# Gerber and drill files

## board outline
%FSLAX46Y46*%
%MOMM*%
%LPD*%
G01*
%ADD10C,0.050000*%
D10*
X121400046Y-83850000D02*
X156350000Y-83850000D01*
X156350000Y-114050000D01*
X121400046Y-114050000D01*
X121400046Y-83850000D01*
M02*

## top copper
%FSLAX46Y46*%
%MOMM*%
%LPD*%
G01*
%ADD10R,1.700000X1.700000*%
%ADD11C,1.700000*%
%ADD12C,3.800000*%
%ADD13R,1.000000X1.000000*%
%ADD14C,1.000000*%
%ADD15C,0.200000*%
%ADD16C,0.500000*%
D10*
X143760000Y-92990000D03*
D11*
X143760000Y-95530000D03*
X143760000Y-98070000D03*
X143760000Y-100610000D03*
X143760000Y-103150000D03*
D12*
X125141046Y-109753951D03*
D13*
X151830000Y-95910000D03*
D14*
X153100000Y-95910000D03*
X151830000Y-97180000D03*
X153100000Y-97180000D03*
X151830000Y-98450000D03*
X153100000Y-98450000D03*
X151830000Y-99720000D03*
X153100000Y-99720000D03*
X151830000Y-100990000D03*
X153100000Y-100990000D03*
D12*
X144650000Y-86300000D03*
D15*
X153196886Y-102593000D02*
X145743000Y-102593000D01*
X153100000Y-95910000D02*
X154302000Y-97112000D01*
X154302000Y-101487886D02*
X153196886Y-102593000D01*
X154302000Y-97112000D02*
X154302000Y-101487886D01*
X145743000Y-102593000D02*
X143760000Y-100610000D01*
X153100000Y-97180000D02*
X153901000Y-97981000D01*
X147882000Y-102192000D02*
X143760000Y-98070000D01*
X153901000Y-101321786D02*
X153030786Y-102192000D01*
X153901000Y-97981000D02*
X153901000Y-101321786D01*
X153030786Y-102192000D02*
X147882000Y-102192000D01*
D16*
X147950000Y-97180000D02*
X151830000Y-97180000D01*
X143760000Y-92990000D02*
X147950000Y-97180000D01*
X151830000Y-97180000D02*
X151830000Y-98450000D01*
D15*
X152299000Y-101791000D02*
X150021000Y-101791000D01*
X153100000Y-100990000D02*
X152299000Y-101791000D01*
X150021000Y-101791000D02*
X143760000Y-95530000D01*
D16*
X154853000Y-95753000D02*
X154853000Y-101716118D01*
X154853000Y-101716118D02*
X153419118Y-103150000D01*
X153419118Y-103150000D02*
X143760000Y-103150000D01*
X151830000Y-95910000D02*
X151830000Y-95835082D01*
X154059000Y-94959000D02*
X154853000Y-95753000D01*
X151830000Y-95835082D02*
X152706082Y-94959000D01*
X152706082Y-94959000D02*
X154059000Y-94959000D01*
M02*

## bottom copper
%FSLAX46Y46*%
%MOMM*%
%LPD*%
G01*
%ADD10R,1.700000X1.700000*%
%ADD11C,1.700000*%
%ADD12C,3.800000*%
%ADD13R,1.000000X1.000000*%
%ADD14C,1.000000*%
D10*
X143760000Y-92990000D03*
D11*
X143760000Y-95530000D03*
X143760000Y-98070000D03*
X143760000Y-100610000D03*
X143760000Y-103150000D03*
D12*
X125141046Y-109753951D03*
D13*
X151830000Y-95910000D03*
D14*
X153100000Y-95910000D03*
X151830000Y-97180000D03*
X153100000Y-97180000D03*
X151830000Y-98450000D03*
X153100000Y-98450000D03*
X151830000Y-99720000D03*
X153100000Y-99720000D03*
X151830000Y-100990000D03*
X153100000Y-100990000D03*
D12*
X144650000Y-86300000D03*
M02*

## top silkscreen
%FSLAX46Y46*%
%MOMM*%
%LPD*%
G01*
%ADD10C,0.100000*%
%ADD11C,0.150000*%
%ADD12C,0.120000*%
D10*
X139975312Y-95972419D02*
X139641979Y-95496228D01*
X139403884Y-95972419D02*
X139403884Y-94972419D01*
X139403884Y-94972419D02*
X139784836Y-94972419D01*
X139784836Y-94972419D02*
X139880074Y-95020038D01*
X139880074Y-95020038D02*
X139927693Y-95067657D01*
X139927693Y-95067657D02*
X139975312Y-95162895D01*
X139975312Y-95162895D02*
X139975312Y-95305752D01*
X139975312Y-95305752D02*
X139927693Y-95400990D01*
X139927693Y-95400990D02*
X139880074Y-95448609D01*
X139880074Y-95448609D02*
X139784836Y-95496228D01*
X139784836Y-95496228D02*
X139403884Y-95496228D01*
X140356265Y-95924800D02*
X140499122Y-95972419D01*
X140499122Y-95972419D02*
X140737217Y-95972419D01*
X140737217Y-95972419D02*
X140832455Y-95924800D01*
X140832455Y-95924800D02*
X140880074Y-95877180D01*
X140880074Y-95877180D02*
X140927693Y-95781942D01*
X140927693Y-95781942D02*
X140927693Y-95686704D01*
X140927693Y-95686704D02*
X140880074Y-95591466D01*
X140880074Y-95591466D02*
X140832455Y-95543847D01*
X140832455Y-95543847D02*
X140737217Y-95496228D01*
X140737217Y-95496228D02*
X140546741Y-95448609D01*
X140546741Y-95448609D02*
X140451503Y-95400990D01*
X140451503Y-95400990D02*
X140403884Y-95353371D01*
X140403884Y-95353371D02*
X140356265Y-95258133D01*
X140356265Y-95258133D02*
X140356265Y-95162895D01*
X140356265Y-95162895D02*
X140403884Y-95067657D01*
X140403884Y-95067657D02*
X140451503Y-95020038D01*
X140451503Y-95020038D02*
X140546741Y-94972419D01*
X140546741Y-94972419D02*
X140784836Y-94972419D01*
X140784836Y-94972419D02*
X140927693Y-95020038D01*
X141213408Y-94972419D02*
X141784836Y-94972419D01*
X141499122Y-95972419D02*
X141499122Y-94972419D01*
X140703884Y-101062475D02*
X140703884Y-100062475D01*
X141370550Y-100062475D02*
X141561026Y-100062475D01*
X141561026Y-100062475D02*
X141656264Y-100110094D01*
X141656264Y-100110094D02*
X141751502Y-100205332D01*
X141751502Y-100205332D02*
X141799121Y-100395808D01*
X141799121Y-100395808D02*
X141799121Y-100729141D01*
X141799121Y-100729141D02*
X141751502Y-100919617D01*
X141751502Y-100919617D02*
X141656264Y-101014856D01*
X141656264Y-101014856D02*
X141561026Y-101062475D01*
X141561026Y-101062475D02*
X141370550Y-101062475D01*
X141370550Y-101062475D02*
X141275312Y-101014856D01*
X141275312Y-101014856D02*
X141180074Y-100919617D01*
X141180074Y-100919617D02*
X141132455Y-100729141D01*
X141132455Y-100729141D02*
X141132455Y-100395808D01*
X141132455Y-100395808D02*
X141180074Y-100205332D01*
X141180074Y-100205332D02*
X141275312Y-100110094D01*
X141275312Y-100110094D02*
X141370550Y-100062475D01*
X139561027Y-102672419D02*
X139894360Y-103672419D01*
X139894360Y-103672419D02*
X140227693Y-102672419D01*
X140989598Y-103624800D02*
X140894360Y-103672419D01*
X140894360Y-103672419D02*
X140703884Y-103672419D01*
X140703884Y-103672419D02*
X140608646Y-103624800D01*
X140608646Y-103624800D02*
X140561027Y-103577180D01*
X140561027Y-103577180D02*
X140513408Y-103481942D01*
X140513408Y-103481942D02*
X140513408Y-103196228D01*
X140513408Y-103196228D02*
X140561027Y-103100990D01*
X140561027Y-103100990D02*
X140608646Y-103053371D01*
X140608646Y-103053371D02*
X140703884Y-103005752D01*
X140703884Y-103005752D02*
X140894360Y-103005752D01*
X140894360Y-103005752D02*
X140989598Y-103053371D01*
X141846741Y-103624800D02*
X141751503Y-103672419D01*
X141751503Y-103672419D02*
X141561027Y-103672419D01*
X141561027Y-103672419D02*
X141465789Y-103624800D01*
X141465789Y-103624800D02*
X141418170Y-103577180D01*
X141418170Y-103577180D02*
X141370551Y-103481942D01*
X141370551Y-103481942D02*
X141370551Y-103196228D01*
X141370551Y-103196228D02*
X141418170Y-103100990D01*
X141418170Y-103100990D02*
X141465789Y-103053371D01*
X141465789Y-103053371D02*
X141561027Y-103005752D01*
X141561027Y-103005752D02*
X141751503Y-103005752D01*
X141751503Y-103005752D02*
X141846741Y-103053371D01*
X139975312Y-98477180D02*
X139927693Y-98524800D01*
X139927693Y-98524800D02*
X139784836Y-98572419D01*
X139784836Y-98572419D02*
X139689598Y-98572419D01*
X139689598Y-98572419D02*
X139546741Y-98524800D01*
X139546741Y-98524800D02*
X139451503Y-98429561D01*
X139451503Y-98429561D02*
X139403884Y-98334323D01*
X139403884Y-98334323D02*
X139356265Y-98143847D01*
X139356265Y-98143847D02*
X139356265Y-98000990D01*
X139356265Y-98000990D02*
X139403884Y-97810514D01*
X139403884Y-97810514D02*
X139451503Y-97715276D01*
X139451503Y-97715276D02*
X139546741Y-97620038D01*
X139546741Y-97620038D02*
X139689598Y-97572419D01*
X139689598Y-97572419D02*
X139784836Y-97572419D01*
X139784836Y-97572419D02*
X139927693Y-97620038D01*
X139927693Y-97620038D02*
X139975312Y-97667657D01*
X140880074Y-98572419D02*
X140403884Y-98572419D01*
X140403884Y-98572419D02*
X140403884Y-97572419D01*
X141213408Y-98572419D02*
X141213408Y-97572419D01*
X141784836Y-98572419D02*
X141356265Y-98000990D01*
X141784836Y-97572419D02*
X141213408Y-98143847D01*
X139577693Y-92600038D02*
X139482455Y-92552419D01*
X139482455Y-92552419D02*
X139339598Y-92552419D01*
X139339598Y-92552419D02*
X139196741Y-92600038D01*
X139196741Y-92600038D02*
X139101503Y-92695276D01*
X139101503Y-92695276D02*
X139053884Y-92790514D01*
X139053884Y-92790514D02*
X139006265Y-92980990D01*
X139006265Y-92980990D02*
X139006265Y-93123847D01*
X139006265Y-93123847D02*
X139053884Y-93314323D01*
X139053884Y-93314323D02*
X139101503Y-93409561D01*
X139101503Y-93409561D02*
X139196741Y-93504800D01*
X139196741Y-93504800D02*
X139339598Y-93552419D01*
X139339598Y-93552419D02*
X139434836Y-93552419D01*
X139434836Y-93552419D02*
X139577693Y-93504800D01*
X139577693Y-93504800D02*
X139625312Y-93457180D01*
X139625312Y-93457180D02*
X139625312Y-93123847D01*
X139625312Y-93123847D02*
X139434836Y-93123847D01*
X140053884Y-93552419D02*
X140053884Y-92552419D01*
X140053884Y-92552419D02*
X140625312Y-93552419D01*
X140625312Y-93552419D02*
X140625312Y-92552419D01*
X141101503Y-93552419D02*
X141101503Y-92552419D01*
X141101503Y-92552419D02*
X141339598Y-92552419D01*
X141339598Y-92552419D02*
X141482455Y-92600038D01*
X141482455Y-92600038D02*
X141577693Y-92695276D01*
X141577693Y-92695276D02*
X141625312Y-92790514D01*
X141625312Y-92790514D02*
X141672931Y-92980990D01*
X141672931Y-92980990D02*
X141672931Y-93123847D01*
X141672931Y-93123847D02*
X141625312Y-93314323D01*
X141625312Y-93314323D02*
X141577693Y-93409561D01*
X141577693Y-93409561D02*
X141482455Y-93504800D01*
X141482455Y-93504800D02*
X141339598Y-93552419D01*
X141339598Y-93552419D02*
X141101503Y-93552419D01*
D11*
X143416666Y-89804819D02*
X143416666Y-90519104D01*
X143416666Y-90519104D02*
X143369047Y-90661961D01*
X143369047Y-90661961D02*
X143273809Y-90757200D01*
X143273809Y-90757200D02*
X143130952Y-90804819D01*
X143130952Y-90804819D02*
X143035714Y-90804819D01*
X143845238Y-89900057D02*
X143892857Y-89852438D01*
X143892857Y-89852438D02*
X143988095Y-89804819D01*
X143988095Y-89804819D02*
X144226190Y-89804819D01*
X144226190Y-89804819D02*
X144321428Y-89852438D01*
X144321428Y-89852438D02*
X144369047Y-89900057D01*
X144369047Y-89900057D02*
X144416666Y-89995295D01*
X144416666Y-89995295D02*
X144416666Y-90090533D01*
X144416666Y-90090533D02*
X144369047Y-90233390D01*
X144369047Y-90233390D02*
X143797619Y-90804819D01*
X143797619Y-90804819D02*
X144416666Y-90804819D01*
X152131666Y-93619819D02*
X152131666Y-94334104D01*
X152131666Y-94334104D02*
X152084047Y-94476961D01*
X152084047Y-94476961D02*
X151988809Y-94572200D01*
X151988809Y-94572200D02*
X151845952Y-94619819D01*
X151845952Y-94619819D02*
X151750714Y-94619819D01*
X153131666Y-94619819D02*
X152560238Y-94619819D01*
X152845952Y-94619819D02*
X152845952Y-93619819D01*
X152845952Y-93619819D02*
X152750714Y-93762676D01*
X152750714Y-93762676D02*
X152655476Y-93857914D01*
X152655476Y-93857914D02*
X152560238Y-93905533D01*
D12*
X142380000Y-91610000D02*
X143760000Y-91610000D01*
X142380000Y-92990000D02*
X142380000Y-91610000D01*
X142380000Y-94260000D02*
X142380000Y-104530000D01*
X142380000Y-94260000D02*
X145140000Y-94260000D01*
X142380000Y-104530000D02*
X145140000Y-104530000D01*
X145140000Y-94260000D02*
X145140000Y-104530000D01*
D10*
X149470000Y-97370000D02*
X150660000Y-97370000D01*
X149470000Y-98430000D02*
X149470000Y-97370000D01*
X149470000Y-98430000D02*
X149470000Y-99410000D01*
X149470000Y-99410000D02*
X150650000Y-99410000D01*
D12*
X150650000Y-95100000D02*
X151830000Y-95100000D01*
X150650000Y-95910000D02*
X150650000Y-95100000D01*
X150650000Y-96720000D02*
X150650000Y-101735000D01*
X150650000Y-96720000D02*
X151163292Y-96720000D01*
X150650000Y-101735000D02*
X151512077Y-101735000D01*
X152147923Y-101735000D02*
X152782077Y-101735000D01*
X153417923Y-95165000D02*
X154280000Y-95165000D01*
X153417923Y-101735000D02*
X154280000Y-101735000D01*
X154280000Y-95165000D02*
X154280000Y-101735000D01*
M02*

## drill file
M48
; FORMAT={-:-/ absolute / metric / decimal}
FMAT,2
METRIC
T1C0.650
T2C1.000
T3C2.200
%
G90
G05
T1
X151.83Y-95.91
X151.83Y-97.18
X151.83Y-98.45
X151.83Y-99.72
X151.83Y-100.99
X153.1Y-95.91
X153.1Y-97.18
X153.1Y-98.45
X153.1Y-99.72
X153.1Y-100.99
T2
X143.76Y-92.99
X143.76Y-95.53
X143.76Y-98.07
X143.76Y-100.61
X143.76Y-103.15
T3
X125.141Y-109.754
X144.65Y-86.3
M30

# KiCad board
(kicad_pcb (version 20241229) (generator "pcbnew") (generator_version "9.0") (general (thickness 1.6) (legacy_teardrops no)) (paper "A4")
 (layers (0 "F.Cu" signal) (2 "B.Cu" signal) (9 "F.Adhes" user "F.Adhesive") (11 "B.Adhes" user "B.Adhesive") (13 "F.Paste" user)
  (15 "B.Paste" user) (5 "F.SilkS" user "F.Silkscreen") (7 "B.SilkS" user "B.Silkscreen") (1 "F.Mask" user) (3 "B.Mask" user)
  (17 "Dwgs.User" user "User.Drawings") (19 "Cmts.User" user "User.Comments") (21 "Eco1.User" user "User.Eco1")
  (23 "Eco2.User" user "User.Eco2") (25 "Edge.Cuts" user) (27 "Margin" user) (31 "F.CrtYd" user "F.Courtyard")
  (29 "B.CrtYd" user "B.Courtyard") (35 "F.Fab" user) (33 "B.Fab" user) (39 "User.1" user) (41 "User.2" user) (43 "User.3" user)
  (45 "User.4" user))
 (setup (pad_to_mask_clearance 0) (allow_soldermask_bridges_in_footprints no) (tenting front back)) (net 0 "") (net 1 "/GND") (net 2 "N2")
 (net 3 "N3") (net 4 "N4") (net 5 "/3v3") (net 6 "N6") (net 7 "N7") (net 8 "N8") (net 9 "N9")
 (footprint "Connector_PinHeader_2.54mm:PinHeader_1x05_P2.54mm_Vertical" (layer "F.Cu") (at 143.76 92.99)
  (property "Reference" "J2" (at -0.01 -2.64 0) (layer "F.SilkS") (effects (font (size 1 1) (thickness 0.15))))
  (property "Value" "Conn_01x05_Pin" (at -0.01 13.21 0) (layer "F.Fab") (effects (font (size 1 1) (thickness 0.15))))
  (fp_line (start -1.38 -1.38) (end 0 -1.38) (stroke (width 0.12) (type solid)) (layer "F.SilkS"))
  (fp_line (start -1.38 0) (end -1.38 -1.38) (stroke (width 0.12) (type solid)) (layer "F.SilkS"))
  (fp_line (start -1.38 1.27) (end -1.38 11.54) (stroke (width 0.12) (type solid)) (layer "F.SilkS"))
  (fp_line (start -1.38 1.27) (end 1.38 1.27) (stroke (width 0.12) (type solid)) (layer "F.SilkS"))
  (fp_line (start -1.38 11.54) (end 1.38 11.54) (stroke (width 0.12) (type solid)) (layer "F.SilkS"))
  (fp_line (start 1.38 1.27) (end 1.38 11.54) (stroke (width 0.12) (type solid)) (layer "F.SilkS"))
  (pad "1" thru_hole rect (at 0 0) (size 1.7 1.7) (drill 1) (layers "*.Cu" "*.Mask") (remove_unused_layers no) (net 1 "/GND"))
  (pad "2" thru_hole circle (at 0 2.54) (size 1.7 1.7) (drill 1) (layers "*.Cu" "*.Mask") (remove_unused_layers no) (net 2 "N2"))
  (pad "3" thru_hole circle (at 0 5.08) (size 1.7 1.7) (drill 1) (layers "*.Cu" "*.Mask") (remove_unused_layers no) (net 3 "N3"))
  (pad "4" thru_hole circle (at 0 7.62) (size 1.7 1.7) (drill 1) (layers "*.Cu" "*.Mask") (remove_unused_layers no) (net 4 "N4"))
  (pad "5" thru_hole circle (at 0 10.16) (size 1.7 1.7) (drill 1) (layers "*.Cu" "*.Mask") (remove_unused_layers no) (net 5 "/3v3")))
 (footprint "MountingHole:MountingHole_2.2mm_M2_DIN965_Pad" (layer "F.Cu") (at 125.141046 109.753951)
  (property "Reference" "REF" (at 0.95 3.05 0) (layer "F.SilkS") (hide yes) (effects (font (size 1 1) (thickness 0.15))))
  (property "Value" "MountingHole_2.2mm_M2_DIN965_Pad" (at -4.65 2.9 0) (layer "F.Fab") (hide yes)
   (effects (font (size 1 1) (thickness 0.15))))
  (pad "1" thru_hole circle (at 0 0) (size 3.8 3.8) (drill 2.2) (layers "*.Cu" "*.Mask") (remove_unused_layers no) (zone_connect 2)))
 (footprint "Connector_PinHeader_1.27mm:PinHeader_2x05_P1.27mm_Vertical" (layer "F.Cu") (at 151.83 95.91)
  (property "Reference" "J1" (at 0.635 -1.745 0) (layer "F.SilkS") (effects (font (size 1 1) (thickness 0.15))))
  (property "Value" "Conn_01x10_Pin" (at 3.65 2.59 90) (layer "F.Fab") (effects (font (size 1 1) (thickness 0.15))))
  (fp_line (start -2.36 1.46) (end -1.17 1.46) (stroke (width 0.1) (type default)) (layer "F.SilkS"))
  (fp_line (start -2.36 2.52) (end -2.36 1.46) (stroke (width 0.1) (type default)) (layer "F.SilkS"))
  (fp_line (start -2.36 2.52) (end -2.36 3.5) (stroke (width 0.1) (type default)) (layer "F.SilkS"))
  (fp_line (start -2.36 3.5) (end -1.18 3.5) (stroke (width 0.1) (type default)) (layer "F.SilkS"))
  (fp_line (start -1.18 -0.81) (end 0 -0.81) (stroke (width 0.12) (type solid)) (layer "F.SilkS"))
  (fp_line (start -1.18 0) (end -1.18 -0.81) (stroke (width 0.12) (type solid)) (layer "F.SilkS"))
  (fp_line (start -1.18 0.81) (end -1.18 5.825) (stroke (width 0.12) (type solid)) (layer "F.SilkS"))
  (fp_line (start -1.18 0.81) (end -0.666708 0.81) (stroke (width 0.12) (type solid)) (layer "F.SilkS"))
  (fp_line (start -1.18 5.825) (end -0.317923 5.825) (stroke (width 0.12) (type solid)) (layer "F.SilkS"))
  (fp_line (start 0.317923 5.825) (end 0.952077 5.825) (stroke (width 0.12) (type solid)) (layer "F.SilkS"))
  (fp_line (start 1.587923 -0.745) (end 2.45 -0.745) (stroke (width 0.12) (type solid)) (layer "F.SilkS"))
  (fp_line (start 1.587923 5.825) (end 2.45 5.825) (stroke (width 0.12) (type solid)) (layer "F.SilkS"))
  (fp_line (start 2.45 -0.745) (end 2.45 5.825) (stroke (width 0.12) (type solid)) (layer "F.SilkS"))
  (pad "1" thru_hole rect (at 0 0) (size 1 1) (drill 0.65) (layers "*.Cu" "*.Mask") (remove_unused_layers no) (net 5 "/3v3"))
  (pad "2" thru_hole circle (at 1.27 0) (size 1 1) (drill 0.65) (layers "*.Cu" "*.Mask") (remove_unused_layers no) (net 4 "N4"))
  (pad "3" thru_hole circle (at 0 1.27) (size 1 1) (drill 0.65) (layers "*.Cu" "*.Mask") (remove_unused_layers no) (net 1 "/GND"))
  (pad "4" thru_hole circle (at 1.27 1.27) (size 1 1) (drill 0.65) (layers "*.Cu" "*.Mask") (remove_unused_layers no) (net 3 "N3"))
  (pad "5" thru_hole circle (at 0 2.54) (size 1 1) (drill 0.65) (layers "*.Cu" "*.Mask") (remove_unused_layers no) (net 1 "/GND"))
  (pad "6" thru_hole circle (at 1.27 2.54) (size 1 1) (drill 0.65) (layers "*.Cu" "*.Mask") (remove_unused_layers no) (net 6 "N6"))
  (pad "7" thru_hole circle (at 0 3.81) (size 1 1) (drill 0.65) (layers "*.Cu" "*.Mask") (remove_unused_layers no) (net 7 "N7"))
  (pad "8" thru_hole circle (at 1.27 3.81) (size 1 1) (drill 0.65) (layers "*.Cu" "*.Mask") (remove_unused_layers no) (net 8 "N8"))
  (pad "9" thru_hole circle (at 0 5.08) (size 1 1) (drill 0.65) (layers "*.Cu" "*.Mask") (remove_unused_layers no) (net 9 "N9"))
  (pad "10" thru_hole circle (at 1.27 5.08) (size 1 1) (drill 0.65) (layers "*.Cu" "*.Mask") (remove_unused_layers no) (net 2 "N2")))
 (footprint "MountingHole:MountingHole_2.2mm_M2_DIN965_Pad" (layer "F.Cu") (at 144.65 86.3)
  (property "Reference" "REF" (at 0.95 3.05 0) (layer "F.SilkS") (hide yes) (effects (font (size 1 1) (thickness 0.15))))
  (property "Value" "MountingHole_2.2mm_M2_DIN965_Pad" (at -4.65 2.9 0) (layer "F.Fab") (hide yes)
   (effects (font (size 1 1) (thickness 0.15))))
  (pad "1" thru_hole circle (at 0 0) (size 3.8 3.8) (drill 2.2) (layers "*.Cu" "*.Mask") (remove_unused_layers no) (zone_connect 2)))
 (gr_rect (start 121.400046 83.85) (end 156.35 114.05) (stroke (width 0.05) (type solid)) (fill no) (layer "Edge.Cuts"))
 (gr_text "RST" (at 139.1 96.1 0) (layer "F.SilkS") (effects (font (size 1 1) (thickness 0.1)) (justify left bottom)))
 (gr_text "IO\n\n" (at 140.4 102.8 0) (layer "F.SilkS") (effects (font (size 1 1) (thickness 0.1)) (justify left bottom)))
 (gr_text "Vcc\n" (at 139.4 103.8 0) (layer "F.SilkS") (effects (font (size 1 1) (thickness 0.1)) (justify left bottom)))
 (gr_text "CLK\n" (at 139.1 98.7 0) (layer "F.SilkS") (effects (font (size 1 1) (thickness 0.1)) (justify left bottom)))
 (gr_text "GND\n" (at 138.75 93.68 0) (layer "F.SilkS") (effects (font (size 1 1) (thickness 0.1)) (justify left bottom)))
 (segment (start 153.196886 102.593) (end 145.743 102.593) (width 0.2) (layer "F.Cu") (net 4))
 (segment (start 153.1 95.91) (end 154.302 97.112) (width 0.2) (layer "F.Cu") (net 4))
 (segment (start 154.302 101.487886) (end 153.196886 102.593) (width 0.2) (layer "F.Cu") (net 4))
 (segment (start 154.302 97.112) (end 154.302 101.487886) (width 0.2) (layer "F.Cu") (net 4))
 (segment (start 145.743 102.593) (end 143.76 100.61) (width 0.2) (layer "F.Cu") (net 4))
 (segment (start 153.1 97.18) (end 153.901 97.981) (width 0.2) (layer "F.Cu") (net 3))
 (segment (start 147.882 102.192) (end 143.76 98.07) (width 0.2) (layer "F.Cu") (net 3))
 (segment (start 153.901 101.321786) (end 153.030786 102.192) (width 0.2) (layer "F.Cu") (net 3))
 (segment (start 153.901 97.981) (end 153.901 101.321786) (width 0.2) (layer "F.Cu") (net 3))
 (segment (start 153.030786 102.192) (end 147.882 102.192) (width 0.2) (layer "F.Cu") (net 3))
 (segment (start 147.95 97.18) (end 151.83 97.18) (width 0.5) (layer "F.Cu") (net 1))
 (segment (start 143.76 92.99) (end 147.95 97.18) (width 0.5) (layer "F.Cu") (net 1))
 (segment (start 151.83 97.18) (end 151.83 98.45) (width 0.5) (layer "F.Cu") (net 1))
 (segment (start 152.299 101.791) (end 150.021 101.791) (width 0.2) (layer "F.Cu") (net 2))
 (segment (start 153.1 100.99) (end 152.299 101.791) (width 0.2) (layer "F.Cu") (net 2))
 (segment (start 150.021 101.791) (end 143.76 95.53) (width 0.2) (layer "F.Cu") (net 2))
 (segment (start 154.853 95.753) (end 154.853 101.716118) (width 0.5) (layer "F.Cu") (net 5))
 (segment (start 154.853 101.716118) (end 153.419118 103.15) (width 0.5) (layer "F.Cu") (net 5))
 (segment (start 153.419118 103.15) (end 143.76 103.15) (width 0.5) (layer "F.Cu") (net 5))
 (segment (start 151.83 95.91) (end 151.83 95.835082) (width 0.5) (layer "F.Cu") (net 5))
 (segment (start 154.059 94.959) (end 154.853 95.753) (width 0.5) (layer "F.Cu") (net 5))
 (segment (start 151.83 95.835082) (end 152.706082 94.959) (width 0.5) (layer "F.Cu") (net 5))
 (segment (start 152.706082 94.959) (end 154.059 94.959) (width 0.5) (layer "F.Cu") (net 5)))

